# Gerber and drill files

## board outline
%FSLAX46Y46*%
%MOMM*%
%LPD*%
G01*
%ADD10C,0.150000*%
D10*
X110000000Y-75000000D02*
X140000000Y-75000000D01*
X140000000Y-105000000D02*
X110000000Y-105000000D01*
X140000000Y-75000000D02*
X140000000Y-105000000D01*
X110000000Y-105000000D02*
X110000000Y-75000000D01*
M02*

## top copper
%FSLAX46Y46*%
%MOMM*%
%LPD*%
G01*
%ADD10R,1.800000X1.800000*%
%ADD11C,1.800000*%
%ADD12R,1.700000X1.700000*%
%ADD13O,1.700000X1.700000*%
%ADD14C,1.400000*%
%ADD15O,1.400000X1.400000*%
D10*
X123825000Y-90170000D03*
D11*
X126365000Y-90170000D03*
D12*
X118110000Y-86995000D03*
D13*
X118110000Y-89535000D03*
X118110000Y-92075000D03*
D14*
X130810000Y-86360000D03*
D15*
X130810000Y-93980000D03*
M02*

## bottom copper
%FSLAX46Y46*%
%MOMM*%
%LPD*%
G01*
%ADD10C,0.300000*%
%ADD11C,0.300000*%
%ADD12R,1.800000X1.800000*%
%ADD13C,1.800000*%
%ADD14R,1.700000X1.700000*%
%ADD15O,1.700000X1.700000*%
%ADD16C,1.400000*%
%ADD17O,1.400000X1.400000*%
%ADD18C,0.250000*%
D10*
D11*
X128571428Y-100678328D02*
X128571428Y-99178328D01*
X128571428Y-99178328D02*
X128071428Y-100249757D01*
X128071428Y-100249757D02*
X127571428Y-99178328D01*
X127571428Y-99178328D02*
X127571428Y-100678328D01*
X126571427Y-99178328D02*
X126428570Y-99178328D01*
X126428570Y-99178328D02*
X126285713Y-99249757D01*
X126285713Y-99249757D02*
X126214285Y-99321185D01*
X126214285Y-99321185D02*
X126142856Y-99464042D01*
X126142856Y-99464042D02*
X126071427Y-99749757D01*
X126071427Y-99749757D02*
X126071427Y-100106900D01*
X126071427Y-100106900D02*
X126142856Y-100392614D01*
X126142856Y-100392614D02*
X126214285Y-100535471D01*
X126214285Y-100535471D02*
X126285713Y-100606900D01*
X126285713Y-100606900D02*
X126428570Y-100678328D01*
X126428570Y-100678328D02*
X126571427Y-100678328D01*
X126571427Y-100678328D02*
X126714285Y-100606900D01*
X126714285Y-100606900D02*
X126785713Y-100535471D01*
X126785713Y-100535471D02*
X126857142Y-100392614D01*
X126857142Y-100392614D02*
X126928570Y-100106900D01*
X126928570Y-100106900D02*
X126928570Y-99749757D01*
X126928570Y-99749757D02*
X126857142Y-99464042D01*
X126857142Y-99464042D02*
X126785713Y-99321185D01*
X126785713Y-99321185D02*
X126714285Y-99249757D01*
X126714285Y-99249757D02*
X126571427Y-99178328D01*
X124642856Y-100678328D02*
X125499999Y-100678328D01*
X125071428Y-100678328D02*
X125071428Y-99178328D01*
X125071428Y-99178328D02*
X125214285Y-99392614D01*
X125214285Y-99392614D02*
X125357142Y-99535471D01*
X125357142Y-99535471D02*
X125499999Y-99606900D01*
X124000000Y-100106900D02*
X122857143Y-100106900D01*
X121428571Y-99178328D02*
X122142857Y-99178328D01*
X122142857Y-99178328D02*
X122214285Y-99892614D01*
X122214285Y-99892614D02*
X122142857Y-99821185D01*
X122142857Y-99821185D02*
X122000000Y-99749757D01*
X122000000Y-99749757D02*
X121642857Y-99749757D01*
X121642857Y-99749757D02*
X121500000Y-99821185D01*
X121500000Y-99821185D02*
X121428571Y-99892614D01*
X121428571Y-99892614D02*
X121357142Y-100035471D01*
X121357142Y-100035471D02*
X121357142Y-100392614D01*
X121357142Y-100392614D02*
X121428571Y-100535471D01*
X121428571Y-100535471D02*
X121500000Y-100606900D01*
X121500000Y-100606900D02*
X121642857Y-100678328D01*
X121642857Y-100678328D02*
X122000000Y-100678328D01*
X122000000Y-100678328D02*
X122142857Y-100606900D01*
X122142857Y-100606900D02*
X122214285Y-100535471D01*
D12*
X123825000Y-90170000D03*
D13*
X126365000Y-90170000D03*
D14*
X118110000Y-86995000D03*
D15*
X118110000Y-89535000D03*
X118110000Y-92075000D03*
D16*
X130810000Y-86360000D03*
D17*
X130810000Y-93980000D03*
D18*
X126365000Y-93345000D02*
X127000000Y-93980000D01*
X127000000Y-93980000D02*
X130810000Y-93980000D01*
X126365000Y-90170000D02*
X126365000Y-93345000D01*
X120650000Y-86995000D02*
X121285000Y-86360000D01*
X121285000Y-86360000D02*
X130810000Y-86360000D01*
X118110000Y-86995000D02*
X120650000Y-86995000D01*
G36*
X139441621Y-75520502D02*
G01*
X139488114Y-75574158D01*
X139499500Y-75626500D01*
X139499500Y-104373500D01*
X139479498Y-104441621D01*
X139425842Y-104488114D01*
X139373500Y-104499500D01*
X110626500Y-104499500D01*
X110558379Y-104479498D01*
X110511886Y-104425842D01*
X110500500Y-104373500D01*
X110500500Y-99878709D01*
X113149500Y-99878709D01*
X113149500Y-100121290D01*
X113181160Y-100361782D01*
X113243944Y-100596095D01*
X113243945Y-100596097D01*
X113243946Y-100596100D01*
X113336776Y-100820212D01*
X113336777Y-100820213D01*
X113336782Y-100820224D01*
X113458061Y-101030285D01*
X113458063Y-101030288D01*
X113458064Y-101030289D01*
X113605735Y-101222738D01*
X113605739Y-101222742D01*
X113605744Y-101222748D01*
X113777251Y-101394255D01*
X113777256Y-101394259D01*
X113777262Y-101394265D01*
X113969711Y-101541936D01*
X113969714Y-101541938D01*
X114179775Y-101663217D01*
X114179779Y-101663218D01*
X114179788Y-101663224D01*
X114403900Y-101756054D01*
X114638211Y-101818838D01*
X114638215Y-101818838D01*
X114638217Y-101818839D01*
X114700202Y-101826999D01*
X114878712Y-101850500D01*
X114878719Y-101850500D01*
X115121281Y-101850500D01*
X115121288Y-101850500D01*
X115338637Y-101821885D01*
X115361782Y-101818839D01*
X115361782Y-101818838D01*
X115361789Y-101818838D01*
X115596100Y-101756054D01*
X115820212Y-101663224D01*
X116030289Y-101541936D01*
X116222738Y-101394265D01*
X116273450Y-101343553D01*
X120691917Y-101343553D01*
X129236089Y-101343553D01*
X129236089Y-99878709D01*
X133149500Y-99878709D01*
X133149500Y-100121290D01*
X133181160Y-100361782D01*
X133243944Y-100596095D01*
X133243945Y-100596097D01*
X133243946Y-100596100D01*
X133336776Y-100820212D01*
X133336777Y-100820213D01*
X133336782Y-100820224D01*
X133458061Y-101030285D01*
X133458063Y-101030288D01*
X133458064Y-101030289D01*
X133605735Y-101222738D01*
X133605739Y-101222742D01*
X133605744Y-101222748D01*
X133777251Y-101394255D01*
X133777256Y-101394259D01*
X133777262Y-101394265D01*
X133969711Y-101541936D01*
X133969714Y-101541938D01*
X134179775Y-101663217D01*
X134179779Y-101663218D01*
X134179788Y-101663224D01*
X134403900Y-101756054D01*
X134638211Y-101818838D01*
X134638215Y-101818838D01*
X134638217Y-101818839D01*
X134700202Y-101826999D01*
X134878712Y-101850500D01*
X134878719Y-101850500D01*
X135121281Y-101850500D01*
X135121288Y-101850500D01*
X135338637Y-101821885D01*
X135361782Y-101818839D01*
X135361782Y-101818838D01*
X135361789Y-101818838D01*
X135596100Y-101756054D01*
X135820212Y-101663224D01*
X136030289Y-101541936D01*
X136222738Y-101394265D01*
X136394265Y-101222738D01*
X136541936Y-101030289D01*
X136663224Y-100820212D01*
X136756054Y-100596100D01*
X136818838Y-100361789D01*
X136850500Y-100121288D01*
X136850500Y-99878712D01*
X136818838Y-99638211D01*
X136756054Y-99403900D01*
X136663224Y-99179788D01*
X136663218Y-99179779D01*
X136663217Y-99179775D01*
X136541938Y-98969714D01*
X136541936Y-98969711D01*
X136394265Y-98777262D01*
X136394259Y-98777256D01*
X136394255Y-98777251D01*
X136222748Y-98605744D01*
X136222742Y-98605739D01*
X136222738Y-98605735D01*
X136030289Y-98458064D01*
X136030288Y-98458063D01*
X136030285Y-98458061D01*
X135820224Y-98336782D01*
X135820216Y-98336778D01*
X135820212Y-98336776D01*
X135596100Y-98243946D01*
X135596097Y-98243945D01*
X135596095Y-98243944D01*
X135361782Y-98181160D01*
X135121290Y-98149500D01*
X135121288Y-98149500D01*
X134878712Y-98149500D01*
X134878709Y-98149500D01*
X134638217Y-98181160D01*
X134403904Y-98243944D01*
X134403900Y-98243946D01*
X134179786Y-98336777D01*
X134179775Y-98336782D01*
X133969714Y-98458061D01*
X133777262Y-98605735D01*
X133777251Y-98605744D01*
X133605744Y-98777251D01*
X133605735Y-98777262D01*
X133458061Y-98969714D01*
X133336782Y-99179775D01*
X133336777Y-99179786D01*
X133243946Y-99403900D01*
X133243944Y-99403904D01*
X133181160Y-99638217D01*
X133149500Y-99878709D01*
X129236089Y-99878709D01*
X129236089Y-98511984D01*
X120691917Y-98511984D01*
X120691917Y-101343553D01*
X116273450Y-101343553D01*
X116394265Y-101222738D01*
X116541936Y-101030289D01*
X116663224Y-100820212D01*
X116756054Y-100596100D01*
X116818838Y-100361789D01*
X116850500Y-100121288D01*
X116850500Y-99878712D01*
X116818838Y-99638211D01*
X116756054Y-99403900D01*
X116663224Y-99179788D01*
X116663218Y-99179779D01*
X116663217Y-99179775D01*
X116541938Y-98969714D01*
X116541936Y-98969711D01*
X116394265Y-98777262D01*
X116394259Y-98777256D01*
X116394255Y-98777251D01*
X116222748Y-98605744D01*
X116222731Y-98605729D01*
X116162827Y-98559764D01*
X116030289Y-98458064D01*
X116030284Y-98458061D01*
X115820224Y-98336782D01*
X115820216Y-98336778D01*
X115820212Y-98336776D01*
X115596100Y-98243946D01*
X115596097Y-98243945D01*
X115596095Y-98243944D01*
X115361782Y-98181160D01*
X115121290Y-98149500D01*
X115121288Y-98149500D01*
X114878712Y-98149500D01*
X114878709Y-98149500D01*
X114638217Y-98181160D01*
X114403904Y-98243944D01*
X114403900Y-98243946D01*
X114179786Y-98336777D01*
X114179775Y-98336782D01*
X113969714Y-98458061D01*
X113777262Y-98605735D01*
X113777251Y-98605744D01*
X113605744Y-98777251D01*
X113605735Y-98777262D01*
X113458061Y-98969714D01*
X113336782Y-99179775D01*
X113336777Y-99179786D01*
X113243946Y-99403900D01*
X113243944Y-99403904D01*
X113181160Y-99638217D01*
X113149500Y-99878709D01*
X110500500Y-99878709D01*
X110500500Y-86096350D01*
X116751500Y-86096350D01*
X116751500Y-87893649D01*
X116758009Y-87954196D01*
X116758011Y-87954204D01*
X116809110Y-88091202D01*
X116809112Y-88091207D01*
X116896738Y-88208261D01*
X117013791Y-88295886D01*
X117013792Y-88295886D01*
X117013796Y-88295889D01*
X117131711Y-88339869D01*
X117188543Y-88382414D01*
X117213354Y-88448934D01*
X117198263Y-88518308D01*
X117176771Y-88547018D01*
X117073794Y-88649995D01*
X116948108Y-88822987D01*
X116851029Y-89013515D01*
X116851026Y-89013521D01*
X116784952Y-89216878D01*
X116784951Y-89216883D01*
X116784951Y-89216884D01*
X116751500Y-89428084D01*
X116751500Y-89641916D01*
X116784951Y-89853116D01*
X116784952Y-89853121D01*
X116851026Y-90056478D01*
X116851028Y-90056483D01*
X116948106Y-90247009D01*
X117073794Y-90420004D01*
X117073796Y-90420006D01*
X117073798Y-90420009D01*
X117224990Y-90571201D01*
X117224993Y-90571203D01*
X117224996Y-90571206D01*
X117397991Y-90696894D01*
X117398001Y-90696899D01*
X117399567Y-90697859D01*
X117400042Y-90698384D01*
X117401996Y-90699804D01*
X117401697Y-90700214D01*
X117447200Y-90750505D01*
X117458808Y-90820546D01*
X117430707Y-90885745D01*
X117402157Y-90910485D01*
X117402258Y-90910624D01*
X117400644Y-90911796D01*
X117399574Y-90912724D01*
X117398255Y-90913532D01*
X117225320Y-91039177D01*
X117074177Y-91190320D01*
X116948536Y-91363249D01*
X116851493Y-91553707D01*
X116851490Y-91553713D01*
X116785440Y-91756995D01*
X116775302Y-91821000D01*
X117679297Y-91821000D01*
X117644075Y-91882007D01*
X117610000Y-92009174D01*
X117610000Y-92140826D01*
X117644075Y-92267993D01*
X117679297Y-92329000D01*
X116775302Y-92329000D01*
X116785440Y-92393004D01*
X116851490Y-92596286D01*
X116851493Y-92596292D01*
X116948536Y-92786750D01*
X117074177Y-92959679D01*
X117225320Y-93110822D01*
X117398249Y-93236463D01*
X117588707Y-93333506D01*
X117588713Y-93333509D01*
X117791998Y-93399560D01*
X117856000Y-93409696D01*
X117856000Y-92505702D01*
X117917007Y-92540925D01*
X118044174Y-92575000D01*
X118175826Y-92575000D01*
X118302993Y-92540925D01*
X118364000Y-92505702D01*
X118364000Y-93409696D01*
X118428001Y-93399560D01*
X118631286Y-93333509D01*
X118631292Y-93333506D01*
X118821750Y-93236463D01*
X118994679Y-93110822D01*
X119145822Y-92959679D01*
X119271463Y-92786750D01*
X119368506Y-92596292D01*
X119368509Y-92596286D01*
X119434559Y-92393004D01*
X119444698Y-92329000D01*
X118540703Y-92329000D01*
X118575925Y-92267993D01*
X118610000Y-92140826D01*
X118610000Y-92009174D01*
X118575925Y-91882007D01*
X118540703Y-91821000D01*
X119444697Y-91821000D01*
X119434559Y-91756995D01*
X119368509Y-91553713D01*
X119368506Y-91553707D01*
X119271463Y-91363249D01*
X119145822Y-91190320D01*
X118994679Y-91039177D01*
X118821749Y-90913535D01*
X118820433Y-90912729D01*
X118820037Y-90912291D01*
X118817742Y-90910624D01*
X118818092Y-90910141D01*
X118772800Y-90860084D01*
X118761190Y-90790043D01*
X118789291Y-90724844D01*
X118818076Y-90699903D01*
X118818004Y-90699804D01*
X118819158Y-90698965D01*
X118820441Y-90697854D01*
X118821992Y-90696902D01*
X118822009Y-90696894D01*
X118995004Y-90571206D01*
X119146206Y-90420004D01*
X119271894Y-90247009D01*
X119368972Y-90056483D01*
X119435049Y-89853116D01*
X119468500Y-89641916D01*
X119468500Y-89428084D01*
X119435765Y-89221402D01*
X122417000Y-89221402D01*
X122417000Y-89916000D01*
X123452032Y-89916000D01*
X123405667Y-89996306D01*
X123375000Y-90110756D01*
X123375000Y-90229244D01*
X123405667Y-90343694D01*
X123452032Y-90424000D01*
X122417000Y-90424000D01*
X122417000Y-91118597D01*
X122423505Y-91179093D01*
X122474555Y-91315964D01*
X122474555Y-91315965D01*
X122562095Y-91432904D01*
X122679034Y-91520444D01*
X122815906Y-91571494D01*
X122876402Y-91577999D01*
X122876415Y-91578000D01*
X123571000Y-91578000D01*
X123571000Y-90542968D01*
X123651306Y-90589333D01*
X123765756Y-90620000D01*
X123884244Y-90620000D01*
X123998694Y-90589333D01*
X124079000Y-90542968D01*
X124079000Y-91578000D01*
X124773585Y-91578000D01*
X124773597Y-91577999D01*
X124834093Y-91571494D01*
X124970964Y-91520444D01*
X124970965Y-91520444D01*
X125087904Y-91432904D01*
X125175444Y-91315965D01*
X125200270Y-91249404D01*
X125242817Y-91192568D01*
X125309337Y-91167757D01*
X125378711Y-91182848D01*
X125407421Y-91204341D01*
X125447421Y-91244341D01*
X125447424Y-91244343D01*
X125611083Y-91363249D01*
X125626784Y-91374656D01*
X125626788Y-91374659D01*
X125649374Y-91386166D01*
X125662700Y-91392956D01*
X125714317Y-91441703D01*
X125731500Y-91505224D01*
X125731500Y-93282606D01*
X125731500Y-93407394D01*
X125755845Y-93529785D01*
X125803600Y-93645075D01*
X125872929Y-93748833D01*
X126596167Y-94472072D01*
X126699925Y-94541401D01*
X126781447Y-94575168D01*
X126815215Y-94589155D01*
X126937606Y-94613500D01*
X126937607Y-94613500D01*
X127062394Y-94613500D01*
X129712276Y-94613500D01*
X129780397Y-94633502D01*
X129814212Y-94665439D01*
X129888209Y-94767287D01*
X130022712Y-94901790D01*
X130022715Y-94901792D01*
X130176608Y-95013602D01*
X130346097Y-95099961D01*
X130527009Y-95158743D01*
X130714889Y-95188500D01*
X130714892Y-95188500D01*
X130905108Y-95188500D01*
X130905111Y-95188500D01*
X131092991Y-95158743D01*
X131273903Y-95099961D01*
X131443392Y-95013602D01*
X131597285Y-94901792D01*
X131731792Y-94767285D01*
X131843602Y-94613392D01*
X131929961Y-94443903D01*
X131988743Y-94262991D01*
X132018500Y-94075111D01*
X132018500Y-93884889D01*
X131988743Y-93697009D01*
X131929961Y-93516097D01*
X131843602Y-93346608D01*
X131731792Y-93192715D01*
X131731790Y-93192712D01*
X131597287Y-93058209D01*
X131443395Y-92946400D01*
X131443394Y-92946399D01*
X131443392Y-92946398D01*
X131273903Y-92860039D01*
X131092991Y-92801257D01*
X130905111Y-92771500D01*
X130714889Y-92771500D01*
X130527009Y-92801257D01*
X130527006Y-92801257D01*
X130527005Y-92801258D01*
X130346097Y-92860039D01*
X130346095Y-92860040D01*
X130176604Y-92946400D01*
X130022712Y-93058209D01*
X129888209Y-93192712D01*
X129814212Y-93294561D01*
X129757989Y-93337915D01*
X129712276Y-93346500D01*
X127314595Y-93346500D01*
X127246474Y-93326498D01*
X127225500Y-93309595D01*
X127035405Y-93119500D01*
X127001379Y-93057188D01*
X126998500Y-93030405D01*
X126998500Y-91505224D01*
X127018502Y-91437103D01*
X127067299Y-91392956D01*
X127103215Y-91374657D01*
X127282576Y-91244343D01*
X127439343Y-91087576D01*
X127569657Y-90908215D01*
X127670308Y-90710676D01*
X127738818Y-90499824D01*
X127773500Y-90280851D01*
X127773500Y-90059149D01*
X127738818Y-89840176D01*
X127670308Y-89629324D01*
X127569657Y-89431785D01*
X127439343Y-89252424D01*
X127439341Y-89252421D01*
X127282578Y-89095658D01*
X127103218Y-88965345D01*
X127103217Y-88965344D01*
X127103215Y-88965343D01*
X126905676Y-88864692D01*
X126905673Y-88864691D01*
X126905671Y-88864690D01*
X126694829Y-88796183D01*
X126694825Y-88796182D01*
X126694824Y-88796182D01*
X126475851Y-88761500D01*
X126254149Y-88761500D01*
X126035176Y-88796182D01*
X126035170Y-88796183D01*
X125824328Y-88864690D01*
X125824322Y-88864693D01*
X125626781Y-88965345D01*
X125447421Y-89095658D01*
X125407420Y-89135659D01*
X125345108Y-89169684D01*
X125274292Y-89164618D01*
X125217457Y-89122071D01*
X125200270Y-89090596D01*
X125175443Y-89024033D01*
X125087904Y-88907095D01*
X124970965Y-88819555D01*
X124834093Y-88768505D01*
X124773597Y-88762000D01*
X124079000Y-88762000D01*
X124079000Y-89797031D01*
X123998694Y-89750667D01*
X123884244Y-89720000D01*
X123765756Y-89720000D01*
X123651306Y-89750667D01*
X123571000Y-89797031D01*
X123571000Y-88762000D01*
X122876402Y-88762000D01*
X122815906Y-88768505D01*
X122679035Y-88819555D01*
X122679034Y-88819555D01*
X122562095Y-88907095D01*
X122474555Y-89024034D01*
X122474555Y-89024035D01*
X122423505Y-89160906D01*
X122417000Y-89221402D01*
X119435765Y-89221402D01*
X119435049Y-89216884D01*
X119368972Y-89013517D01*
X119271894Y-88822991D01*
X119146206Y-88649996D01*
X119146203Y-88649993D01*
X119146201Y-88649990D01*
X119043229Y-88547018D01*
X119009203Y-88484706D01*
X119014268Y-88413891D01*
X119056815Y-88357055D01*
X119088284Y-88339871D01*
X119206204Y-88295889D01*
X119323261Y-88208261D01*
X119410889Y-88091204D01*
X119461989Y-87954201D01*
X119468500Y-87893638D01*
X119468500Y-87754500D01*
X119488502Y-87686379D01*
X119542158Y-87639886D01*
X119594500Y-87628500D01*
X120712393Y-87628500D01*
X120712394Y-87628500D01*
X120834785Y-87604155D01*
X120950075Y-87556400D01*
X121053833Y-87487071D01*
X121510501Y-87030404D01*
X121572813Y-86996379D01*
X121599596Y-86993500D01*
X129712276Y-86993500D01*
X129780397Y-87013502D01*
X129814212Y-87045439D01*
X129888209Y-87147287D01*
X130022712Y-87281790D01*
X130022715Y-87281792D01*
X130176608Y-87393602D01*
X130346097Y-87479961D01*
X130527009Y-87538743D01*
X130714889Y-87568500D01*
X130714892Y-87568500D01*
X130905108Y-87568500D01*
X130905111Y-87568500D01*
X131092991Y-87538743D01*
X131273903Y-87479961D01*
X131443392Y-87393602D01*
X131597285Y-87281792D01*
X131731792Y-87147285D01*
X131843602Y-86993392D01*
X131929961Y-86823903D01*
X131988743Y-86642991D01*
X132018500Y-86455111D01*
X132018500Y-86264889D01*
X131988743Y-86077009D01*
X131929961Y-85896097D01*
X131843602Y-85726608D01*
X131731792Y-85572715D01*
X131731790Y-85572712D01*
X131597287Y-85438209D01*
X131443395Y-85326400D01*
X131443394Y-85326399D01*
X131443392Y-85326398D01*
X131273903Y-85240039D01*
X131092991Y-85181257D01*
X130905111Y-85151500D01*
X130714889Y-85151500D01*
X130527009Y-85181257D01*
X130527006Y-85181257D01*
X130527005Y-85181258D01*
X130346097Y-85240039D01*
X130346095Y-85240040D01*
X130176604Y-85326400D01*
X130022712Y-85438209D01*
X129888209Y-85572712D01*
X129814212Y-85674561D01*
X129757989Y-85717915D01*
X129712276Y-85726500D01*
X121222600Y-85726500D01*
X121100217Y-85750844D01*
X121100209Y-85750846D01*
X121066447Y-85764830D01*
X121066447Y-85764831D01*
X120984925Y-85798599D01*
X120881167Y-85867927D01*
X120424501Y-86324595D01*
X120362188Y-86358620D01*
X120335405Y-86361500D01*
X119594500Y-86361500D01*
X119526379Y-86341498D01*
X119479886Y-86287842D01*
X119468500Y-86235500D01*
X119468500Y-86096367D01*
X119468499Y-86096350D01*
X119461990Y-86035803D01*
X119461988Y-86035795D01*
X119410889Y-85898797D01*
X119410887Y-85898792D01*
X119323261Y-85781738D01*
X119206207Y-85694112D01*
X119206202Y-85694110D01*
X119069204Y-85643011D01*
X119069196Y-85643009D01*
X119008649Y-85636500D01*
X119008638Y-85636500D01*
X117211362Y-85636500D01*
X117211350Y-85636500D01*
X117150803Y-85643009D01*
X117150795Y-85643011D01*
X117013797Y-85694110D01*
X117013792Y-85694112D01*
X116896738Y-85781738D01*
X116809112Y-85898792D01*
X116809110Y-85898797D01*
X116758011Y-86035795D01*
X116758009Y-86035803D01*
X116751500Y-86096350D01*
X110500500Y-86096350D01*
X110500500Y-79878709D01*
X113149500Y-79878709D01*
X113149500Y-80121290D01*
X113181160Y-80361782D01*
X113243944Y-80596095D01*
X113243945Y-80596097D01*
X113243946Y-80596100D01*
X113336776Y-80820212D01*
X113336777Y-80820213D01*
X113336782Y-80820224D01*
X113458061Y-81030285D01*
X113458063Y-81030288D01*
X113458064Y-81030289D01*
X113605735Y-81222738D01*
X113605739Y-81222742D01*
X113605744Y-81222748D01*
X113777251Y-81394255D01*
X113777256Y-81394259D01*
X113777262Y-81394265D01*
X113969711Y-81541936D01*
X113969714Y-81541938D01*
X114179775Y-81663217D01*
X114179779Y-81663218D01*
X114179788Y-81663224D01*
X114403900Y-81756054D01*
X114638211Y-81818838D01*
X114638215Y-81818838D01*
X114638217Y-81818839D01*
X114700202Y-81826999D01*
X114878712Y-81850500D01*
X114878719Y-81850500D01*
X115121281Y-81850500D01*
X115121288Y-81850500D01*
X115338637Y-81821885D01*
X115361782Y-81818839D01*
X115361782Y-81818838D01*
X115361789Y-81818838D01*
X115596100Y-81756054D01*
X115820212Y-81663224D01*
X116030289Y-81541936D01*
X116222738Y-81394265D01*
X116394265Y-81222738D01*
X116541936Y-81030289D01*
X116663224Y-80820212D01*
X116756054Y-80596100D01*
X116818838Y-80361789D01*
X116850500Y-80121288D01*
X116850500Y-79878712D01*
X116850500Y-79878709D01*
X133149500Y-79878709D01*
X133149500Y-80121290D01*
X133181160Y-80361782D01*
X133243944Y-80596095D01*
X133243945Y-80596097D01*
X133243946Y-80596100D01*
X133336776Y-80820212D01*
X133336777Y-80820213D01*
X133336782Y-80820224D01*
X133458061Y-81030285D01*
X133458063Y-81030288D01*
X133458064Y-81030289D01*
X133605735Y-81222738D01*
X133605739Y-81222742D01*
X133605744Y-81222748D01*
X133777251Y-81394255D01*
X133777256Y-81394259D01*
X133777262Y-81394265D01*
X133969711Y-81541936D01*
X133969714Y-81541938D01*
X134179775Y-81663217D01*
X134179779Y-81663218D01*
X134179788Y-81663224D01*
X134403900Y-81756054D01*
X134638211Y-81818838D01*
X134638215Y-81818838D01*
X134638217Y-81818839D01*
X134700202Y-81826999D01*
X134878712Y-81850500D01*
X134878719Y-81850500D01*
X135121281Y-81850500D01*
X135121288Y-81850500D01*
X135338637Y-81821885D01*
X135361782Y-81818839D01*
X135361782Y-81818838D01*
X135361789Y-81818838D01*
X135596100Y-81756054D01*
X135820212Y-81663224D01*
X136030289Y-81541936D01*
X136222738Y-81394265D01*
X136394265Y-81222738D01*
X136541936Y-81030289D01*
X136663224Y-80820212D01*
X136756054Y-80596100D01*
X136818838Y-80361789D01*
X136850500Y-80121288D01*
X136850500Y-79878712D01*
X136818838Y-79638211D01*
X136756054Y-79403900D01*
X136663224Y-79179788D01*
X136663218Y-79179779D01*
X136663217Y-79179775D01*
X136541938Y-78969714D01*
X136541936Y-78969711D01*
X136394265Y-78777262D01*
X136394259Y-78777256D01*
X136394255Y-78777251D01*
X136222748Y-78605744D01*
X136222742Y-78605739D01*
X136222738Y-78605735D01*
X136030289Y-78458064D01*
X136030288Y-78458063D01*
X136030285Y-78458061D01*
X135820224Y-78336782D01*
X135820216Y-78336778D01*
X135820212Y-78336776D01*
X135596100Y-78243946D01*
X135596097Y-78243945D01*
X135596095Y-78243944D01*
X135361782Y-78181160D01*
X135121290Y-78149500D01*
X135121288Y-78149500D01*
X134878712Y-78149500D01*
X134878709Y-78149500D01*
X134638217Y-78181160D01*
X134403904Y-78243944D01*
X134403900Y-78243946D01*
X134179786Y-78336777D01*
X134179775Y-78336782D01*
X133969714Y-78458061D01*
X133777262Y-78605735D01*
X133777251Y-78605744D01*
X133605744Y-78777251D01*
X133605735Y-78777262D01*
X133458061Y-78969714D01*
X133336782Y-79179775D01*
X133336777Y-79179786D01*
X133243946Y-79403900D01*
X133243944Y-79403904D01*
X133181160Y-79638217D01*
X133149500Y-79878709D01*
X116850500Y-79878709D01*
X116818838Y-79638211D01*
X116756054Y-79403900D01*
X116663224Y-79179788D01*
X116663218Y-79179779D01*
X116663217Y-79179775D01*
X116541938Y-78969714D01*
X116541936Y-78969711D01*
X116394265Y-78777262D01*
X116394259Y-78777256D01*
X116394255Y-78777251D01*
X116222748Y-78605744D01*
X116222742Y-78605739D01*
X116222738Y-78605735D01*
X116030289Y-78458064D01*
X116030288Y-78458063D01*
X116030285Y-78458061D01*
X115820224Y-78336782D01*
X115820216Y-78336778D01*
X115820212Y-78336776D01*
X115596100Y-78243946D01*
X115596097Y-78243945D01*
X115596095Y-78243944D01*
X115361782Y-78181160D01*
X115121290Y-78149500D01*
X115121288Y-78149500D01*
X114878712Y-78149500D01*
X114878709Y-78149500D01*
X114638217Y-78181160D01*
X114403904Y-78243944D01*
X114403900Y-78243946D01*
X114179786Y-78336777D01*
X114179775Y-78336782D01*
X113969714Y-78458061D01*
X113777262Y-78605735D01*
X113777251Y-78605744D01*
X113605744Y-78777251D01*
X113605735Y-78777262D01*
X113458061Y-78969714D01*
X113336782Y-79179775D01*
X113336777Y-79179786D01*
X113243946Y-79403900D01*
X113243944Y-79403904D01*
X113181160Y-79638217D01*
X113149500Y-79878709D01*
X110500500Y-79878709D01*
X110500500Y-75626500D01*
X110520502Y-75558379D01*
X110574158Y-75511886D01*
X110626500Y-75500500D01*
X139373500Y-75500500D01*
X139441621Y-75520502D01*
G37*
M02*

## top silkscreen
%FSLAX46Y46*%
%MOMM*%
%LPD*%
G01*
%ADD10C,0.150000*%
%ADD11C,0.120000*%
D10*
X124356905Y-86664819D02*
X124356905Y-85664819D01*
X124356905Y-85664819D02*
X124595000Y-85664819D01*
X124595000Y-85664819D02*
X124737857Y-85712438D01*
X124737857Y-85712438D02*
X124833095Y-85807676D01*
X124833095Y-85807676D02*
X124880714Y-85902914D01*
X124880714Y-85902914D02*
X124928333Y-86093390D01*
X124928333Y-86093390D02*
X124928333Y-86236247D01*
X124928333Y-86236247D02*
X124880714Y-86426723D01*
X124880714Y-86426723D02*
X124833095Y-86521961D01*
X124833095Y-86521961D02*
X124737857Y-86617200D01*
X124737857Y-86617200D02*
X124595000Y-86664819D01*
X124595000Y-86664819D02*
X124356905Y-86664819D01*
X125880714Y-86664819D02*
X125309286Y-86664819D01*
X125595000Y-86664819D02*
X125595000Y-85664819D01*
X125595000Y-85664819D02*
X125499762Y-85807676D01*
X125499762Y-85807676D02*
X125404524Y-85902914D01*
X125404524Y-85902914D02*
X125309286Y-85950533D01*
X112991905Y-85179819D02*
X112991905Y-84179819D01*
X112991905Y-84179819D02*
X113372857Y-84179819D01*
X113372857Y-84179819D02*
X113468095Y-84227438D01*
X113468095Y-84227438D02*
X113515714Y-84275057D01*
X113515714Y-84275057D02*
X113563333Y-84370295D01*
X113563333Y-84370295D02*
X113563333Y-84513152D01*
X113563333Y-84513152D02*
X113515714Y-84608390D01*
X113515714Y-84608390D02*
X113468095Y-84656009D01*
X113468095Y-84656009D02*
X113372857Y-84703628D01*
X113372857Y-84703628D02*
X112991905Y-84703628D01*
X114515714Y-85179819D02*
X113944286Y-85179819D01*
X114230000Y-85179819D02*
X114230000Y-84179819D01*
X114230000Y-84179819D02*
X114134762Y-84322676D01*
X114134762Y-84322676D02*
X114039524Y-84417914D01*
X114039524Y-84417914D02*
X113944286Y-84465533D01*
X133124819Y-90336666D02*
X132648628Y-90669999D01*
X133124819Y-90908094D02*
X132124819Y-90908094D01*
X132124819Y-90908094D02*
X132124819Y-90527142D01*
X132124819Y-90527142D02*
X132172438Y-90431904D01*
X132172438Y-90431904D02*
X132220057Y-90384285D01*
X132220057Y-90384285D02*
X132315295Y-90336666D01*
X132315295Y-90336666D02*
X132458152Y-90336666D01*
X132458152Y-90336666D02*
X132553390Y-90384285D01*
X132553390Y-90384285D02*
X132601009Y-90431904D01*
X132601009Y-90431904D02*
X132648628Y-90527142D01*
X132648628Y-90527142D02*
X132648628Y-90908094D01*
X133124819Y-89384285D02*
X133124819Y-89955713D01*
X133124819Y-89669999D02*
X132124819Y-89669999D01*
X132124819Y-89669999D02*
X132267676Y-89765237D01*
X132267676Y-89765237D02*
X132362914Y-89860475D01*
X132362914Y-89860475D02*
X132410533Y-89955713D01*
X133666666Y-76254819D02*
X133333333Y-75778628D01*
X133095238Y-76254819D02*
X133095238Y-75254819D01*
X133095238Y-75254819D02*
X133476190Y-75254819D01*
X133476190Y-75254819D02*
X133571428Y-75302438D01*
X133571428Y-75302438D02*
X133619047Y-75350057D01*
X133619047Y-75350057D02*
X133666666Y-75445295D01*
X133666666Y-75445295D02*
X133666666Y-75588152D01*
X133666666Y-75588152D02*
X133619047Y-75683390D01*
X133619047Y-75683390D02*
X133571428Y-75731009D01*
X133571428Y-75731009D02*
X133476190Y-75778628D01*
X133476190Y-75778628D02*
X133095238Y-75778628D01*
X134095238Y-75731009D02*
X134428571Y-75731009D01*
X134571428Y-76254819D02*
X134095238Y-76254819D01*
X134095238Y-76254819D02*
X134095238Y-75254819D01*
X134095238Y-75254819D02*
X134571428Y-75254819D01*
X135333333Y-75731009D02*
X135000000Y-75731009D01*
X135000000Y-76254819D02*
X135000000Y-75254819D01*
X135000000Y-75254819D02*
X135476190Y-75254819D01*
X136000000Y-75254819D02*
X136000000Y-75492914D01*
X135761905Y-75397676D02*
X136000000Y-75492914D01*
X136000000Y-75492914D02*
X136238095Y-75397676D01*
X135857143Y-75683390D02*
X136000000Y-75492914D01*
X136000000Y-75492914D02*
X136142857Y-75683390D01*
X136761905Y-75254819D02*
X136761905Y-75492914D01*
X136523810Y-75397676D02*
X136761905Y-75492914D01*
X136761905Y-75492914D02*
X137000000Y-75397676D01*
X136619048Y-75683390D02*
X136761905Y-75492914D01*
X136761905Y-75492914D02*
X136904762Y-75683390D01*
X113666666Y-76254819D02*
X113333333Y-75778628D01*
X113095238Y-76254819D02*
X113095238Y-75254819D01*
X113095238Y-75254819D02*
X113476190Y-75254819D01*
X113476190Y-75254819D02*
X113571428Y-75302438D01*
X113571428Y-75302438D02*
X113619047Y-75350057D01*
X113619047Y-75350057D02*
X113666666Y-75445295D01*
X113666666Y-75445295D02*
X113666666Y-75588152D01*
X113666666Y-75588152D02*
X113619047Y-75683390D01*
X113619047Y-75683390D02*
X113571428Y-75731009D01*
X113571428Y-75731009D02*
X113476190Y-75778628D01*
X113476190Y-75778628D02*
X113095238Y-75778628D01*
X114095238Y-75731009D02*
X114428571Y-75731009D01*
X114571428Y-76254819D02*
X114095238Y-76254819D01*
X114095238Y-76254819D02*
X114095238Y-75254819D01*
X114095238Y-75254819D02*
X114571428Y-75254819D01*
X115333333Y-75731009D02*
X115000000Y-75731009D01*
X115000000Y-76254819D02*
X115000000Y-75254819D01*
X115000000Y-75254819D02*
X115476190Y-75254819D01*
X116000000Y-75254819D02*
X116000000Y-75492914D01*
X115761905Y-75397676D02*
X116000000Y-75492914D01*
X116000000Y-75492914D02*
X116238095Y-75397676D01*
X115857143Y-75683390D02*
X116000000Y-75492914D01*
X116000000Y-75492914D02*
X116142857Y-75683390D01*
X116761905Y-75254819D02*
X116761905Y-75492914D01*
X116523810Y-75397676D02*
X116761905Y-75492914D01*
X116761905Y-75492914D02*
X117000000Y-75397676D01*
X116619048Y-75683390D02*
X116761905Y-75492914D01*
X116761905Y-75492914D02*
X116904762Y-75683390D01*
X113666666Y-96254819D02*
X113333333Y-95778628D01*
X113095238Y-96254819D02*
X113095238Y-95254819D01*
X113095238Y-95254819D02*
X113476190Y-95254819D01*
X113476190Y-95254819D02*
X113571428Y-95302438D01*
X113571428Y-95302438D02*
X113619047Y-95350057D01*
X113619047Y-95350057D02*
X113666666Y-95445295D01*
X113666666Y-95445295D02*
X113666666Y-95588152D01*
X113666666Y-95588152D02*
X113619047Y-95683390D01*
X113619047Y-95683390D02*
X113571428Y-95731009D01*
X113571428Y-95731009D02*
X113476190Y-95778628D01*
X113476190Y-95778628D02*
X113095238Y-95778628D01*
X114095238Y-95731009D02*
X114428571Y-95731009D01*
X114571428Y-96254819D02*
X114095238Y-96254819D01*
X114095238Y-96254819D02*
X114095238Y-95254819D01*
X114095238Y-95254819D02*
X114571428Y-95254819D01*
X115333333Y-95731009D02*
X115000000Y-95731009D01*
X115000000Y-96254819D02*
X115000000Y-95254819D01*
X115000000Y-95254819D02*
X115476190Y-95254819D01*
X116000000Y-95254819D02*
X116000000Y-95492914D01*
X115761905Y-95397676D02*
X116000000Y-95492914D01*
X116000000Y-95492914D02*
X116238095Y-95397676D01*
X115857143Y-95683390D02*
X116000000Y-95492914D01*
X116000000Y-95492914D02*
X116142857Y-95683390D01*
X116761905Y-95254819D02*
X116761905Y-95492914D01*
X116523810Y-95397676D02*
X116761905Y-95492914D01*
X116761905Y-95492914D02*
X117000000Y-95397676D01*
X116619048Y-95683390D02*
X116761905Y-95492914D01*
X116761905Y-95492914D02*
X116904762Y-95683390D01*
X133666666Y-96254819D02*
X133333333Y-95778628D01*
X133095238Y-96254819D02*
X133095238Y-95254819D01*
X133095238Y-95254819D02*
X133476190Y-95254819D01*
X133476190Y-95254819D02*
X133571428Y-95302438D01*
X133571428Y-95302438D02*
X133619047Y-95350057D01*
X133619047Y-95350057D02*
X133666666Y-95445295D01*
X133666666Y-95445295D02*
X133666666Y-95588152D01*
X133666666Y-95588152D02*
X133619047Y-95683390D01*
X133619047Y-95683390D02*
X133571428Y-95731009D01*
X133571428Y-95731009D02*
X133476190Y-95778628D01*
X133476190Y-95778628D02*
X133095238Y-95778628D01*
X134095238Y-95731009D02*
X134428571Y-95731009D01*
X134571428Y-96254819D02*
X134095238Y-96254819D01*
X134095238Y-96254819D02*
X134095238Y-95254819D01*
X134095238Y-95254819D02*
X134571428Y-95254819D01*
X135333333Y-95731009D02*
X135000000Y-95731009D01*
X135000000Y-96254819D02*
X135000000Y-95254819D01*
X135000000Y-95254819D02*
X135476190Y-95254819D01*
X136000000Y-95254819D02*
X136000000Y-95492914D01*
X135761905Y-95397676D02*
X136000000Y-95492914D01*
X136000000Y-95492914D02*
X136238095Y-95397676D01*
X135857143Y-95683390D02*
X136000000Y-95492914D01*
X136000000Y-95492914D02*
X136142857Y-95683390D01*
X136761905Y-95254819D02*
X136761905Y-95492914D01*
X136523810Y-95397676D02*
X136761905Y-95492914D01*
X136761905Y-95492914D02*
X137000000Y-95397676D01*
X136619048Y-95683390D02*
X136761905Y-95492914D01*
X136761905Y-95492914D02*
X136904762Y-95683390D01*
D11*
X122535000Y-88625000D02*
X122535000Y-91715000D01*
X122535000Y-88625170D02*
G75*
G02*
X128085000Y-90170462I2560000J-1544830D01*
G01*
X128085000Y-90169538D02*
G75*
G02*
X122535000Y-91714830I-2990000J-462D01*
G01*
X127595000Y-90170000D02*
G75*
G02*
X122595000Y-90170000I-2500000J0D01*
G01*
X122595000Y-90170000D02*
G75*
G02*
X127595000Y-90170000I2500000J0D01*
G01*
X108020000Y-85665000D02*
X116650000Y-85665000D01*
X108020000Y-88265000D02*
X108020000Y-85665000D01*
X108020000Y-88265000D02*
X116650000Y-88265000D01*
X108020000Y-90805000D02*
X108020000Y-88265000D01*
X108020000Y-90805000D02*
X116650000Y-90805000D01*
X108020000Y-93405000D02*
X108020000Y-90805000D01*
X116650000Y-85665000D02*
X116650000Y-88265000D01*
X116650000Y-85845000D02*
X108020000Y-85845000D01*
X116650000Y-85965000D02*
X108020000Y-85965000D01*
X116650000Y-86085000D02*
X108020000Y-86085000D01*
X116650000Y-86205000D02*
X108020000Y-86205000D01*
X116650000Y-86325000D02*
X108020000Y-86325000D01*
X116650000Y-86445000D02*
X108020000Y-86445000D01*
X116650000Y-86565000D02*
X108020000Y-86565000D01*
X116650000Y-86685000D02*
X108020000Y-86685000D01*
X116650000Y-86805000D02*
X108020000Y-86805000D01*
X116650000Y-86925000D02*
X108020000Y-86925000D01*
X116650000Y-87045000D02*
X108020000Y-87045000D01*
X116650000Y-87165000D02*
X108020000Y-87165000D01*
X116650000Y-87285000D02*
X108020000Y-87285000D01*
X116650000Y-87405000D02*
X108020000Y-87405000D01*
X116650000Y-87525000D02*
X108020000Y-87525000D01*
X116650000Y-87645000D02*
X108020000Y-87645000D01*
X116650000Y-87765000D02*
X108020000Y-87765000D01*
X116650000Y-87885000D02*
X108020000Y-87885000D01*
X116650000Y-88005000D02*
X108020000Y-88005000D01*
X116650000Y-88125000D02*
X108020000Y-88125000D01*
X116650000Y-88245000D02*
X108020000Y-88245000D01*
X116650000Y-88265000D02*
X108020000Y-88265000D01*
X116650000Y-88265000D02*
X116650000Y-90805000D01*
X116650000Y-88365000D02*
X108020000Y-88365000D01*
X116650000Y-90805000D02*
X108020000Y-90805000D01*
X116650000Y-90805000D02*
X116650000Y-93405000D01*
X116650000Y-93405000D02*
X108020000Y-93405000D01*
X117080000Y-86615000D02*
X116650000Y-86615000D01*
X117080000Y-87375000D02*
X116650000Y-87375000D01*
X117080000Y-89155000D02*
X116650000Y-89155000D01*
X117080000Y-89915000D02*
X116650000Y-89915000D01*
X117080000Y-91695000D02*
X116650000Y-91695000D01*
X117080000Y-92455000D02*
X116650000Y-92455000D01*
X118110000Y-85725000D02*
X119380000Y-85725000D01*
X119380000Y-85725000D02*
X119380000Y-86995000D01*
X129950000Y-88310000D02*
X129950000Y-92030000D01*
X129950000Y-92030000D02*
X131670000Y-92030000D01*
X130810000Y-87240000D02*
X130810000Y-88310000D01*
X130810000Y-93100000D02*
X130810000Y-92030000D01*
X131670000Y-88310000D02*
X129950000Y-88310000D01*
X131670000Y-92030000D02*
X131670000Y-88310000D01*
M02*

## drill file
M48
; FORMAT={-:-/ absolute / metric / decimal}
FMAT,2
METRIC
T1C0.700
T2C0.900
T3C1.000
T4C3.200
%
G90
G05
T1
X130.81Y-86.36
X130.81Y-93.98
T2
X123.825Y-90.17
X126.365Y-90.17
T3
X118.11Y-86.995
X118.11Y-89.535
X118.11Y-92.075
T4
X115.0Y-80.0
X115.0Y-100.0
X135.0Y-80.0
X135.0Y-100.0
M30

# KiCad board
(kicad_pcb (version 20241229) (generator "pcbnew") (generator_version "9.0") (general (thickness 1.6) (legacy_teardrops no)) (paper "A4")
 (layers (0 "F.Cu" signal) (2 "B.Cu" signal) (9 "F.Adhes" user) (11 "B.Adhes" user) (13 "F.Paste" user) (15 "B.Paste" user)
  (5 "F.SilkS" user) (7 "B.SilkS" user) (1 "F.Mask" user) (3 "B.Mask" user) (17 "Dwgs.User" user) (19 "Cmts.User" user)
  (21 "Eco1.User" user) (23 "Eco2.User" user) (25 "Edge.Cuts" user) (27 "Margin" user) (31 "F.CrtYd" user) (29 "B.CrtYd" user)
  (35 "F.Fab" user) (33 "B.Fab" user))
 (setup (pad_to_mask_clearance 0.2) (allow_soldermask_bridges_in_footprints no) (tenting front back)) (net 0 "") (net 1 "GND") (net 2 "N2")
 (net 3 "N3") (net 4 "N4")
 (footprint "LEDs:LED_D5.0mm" (layer "F.Cu") (at 123.825 90.17)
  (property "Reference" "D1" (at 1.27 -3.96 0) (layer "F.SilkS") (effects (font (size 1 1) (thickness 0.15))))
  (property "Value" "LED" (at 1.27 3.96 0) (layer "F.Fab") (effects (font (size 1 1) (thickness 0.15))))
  (fp_line (start -1.29 -1.545) (end -1.29 1.545) (stroke (width 0.12) (type solid)) (layer "F.SilkS"))
  (fp_arc (start -1.29 -1.54483) (mid 2.072002 -2.880433) (end 4.26 0.000462) (stroke (width 0.12) (type solid)) (layer "F.SilkS"))
  (fp_arc (start 4.26 -0.000462) (mid 2.072002 2.880433) (end -1.29 1.54483) (stroke (width 0.12) (type solid)) (layer "F.SilkS"))
  (fp_circle (center 1.27 0) (end 3.77 0) (stroke (width 0.12) (type solid)) (fill no) (layer "F.SilkS"))
  (pad "1" thru_hole rect (at 0 0) (size 1.8 1.8) (drill 0.9) (layers "*.Cu" "*.Mask") (remove_unused_layers no) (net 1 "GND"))
  (pad "2" thru_hole circle (at 2.54 0) (size 1.8 1.8) (drill 0.9) (layers "*.Cu" "*.Mask") (remove_unused_layers no) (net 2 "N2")))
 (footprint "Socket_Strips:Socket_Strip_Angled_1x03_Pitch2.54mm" (layer "F.Cu") (at 118.11 86.995)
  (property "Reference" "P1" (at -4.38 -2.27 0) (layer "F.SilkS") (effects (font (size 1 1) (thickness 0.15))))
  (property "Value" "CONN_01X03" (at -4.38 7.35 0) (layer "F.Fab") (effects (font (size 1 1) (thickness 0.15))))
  (fp_line (start -10.09 -1.33) (end -1.46 -1.33) (stroke (width 0.12) (type solid)) (layer "F.SilkS"))
  (fp_line (start -10.09 1.27) (end -10.09 -1.33) (stroke (width 0.12) (type solid)) (layer "F.SilkS"))
  (fp_line (start -10.09 1.27) (end -1.46 1.27) (stroke (width 0.12) (type solid)) (layer "F.SilkS"))
  (fp_line (start -10.09 3.81) (end -10.09 1.27) (stroke (width 0.12) (type solid)) (layer "F.SilkS"))
  (fp_line (start -10.09 3.81) (end -1.46 3.81) (stroke (width 0.12) (type solid)) (layer "F.SilkS"))
  (fp_line (start -10.09 6.41) (end -10.09 3.81) (stroke (width 0.12) (type solid)) (layer "F.SilkS"))
  (fp_line (start -1.46 -1.33) (end -1.46 1.27) (stroke (width 0.12) (type solid)) (layer "F.SilkS"))
  (fp_line (start -1.46 -1.15) (end -10.09 -1.15) (stroke (width 0.12) (type solid)) (layer "F.SilkS"))
  (fp_line (start -1.46 -1.03) (end -10.09 -1.03) (stroke (width 0.12) (type solid)) (layer "F.SilkS"))
  (fp_line (start -1.46 -0.91) (end -10.09 -0.91) (stroke (width 0.12) (type solid)) (layer "F.SilkS"))
  (fp_line (start -1.46 -0.79) (end -10.09 -0.79) (stroke (width 0.12) (type solid)) (layer "F.SilkS"))
  (fp_line (start -1.46 -0.67) (end -10.09 -0.67) (stroke (width 0.12) (type solid)) (layer "F.SilkS"))
  (fp_line (start -1.46 -0.55) (end -10.09 -0.55) (stroke (width 0.12) (type solid)) (layer "F.SilkS"))
  (fp_line (start -1.46 -0.43) (end -10.09 -0.43) (stroke (width 0.12) (type solid)) (layer "F.SilkS"))
  (fp_line (start -1.46 -0.31) (end -10.09 -0.31) (stroke (width 0.12) (type solid)) (layer "F.SilkS"))
  (fp_line (start -1.46 -0.19) (end -10.09 -0.19) (stroke (width 0.12) (type solid)) (layer "F.SilkS"))
  (fp_line (start -1.46 -0.07) (end -10.09 -0.07) (stroke (width 0.12) (type solid)) (layer "F.SilkS"))
  (fp_line (start -1.46 0.05) (end -10.09 0.05) (stroke (width 0.12) (type solid)) (layer "F.SilkS"))
  (fp_line (start -1.46 0.17) (end -10.09 0.17) (stroke (width 0.12) (type solid)) (layer "F.SilkS"))
  (fp_line (start -1.46 0.29) (end -10.09 0.29) (stroke (width 0.12) (type solid)) (layer "F.SilkS"))
  (fp_line (start -1.46 0.41) (end -10.09 0.41) (stroke (width 0.12) (type solid)) (layer "F.SilkS"))
  (fp_line (start -1.46 0.53) (end -10.09 0.53) (stroke (width 0.12) (type solid)) (layer "F.SilkS"))
  (fp_line (start -1.46 0.65) (end -10.09 0.65) (stroke (width 0.12) (type solid)) (layer "F.SilkS"))
  (fp_line (start -1.46 0.77) (end -10.09 0.77) (stroke (width 0.12) (type solid)) (layer "F.SilkS"))
  (fp_line (start -1.46 0.89) (end -10.09 0.89) (stroke (width 0.12) (type solid)) (layer "F.SilkS"))
  (fp_line (start -1.46 1.01) (end -10.09 1.01) (stroke (width 0.12) (type solid)) (layer "F.SilkS"))
  (fp_line (start -1.46 1.13) (end -10.09 1.13) (stroke (width 0.12) (type solid)) (layer "F.SilkS"))
  (fp_line (start -1.46 1.25) (end -10.09 1.25) (stroke (width 0.12) (type solid)) (layer "F.SilkS"))
  (fp_line (start -1.46 1.27) (end -10.09 1.27) (stroke (width 0.12) (type solid)) (layer "F.SilkS"))
  (fp_line (start -1.46 1.27) (end -1.46 3.81) (stroke (width 0.12) (type solid)) (layer "F.SilkS"))
  (fp_line (start -1.46 1.37) (end -10.09 1.37) (stroke (width 0.12) (type solid)) (layer "F.SilkS"))
  (fp_line (start -1.46 3.81) (end -10.09 3.81) (stroke (width 0.12) (type solid)) (layer "F.SilkS"))
  (fp_line (start -1.46 3.81) (end -1.46 6.41) (stroke (width 0.12) (type solid)) (layer "F.SilkS"))
  (fp_line (start -1.46 6.41) (end -10.09 6.41) (stroke (width 0.12) (type solid)) (layer "F.SilkS"))
  (fp_line (start -1.03 -0.38) (end -1.46 -0.38) (stroke (width 0.12) (type solid)) (layer "F.SilkS"))
  (fp_line (start -1.03 0.38) (end -1.46 0.38) (stroke (width 0.12) (type solid)) (layer "F.SilkS"))
  (fp_line (start -1.03 2.16) (end -1.46 2.16) (stroke (width 0.12) (type solid)) (layer "F.SilkS"))
  (fp_line (start -1.03 2.92) (end -1.46 2.92) (stroke (width 0.12) (type solid)) (layer "F.SilkS"))
  (fp_line (start -1.03 4.7) (end -1.46 4.7) (stroke (width 0.12) (type solid)) (layer "F.SilkS"))
  (fp_line (start -1.03 5.46) (end -1.46 5.46) (stroke (width 0.12) (type solid)) (layer "F.SilkS"))
  (fp_line (start 0 -1.27) (end 1.27 -1.27) (stroke (width 0.12) (type solid)) (layer "F.SilkS"))
  (fp_line (start 1.27 -1.27) (end 1.27 0) (stroke (width 0.12) (type solid)) (layer "F.SilkS"))
  (pad "1" thru_hole rect (at 0 0) (size 1.7 1.7) (drill 1) (layers "*.Cu" "*.Mask") (remove_unused_layers no) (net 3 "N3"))
  (pad "2" thru_hole oval (at 0 2.54) (size 1.7 1.7) (drill 1) (layers "*.Cu" "*.Mask") (remove_unused_layers no) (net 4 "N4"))
  (pad "3" thru_hole oval (at 0 5.08) (size 1.7 1.7) (drill 1) (layers "*.Cu" "*.Mask") (remove_unused_layers no) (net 1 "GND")))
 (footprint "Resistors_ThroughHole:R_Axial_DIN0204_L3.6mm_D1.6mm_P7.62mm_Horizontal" (layer "F.Cu") (at 130.81 86.36 -90)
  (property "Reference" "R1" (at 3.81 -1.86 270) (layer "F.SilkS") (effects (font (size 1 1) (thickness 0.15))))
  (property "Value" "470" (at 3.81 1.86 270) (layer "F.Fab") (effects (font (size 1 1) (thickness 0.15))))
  (fp_line (start 1.95 0.86) (end 5.67 0.86) (stroke (width 0.12) (type solid)) (layer "F.SilkS"))
  (fp_line (start 5.67 0.86) (end 5.67 -0.86) (stroke (width 0.12) (type solid)) (layer "F.SilkS"))
  (fp_line (start 0.88 0) (end 1.95 0) (stroke (width 0.12) (type solid)) (layer "F.SilkS"))
  (fp_line (start 6.74 0) (end 5.67 0) (stroke (width 0.12) (type solid)) (layer "F.SilkS"))
  (fp_line (start 1.95 -0.86) (end 1.95 0.86) (stroke (width 0.12) (type solid)) (layer "F.SilkS"))
  (fp_line (start 5.67 -0.86) (end 1.95 -0.86) (stroke (width 0.12) (type solid)) (layer "F.SilkS"))
  (pad "1" thru_hole circle (at 0 0 270) (size 1.4 1.4) (drill 0.7) (layers "*.Cu" "*.Mask") (remove_unused_layers no) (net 3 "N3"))
  (pad "2" thru_hole oval (at 7.62 0 270) (size 1.4 1.4) (drill 0.7) (layers "*.Cu" "*.Mask") (remove_unused_layers no) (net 2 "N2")))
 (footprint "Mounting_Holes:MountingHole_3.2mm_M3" (layer "F.Cu") (at 135 80)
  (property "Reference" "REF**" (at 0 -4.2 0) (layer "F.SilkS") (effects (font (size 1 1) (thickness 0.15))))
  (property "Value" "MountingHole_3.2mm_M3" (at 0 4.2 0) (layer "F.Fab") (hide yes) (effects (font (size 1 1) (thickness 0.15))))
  (pad "" np_thru_hole circle (at 0 0) (size 3.2 3.2) (drill 3.2) (layers "*.Cu" "*.Mask")))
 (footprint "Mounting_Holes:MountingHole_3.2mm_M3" (layer "F.Cu") (at 115 80)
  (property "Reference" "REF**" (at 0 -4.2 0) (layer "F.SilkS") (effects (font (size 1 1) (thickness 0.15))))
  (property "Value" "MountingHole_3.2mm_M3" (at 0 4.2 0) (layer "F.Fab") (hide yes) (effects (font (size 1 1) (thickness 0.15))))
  (pad "" np_thru_hole circle (at 0 0) (size 3.2 3.2) (drill 3.2) (layers "*.Cu" "*.Mask")))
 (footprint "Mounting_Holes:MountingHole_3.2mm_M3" (layer "F.Cu") (at 115 100)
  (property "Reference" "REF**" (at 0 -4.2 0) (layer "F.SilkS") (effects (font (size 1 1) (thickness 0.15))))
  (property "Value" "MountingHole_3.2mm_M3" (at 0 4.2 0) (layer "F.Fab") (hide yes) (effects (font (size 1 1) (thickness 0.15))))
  (pad "" np_thru_hole circle (at 0 0) (size 3.2 3.2) (drill 3.2) (layers "*.Cu" "*.Mask")))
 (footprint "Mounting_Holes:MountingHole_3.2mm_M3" (layer "F.Cu") (at 135 100)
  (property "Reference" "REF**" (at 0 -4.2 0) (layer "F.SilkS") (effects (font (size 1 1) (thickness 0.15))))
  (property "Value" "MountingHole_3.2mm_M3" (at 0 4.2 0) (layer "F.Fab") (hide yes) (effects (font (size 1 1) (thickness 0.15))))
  (pad "" np_thru_hole circle (at 0 0) (size 3.2 3.2) (drill 3.2) (layers "*.Cu" "*.Mask")))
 (gr_line (start 110 75) (end 140 75) (stroke (width 0.15) (type solid)) (layer "Edge.Cuts"))
 (gr_line (start 140 105) (end 110 105) (stroke (width 0.15) (type solid)) (layer "Edge.Cuts"))
 (gr_line (start 140 75) (end 140 105) (stroke (width 0.15) (type solid)) (layer "Edge.Cuts"))
 (gr_line (start 110 105) (end 110 75) (stroke (width 0.15) (type solid)) (layer "Edge.Cuts"))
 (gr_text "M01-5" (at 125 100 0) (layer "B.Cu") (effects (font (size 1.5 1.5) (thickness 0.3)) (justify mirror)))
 (segment (start 126.365 93.345) (end 127 93.98) (width 0.25) (layer "B.Cu") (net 2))
 (segment (start 127 93.98) (end 130.81 93.98) (width 0.25) (layer "B.Cu") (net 2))
 (segment (start 126.365 90.17) (end 126.365 93.345) (width 0.25) (layer "B.Cu") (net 2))
 (segment (start 120.65 86.995) (end 121.285 86.36) (width 0.25) (layer "B.Cu") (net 3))
 (segment (start 121.285 86.36) (end 130.81 86.36) (width 0.25) (layer "B.Cu") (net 3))
 (segment (start 118.11 86.995) (end 120.65 86.995) (width 0.25) (layer "B.Cu") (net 3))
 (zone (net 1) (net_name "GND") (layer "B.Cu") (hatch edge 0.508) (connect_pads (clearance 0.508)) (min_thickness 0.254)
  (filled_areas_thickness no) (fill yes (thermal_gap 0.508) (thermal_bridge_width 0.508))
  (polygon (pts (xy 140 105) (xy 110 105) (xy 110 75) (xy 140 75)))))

